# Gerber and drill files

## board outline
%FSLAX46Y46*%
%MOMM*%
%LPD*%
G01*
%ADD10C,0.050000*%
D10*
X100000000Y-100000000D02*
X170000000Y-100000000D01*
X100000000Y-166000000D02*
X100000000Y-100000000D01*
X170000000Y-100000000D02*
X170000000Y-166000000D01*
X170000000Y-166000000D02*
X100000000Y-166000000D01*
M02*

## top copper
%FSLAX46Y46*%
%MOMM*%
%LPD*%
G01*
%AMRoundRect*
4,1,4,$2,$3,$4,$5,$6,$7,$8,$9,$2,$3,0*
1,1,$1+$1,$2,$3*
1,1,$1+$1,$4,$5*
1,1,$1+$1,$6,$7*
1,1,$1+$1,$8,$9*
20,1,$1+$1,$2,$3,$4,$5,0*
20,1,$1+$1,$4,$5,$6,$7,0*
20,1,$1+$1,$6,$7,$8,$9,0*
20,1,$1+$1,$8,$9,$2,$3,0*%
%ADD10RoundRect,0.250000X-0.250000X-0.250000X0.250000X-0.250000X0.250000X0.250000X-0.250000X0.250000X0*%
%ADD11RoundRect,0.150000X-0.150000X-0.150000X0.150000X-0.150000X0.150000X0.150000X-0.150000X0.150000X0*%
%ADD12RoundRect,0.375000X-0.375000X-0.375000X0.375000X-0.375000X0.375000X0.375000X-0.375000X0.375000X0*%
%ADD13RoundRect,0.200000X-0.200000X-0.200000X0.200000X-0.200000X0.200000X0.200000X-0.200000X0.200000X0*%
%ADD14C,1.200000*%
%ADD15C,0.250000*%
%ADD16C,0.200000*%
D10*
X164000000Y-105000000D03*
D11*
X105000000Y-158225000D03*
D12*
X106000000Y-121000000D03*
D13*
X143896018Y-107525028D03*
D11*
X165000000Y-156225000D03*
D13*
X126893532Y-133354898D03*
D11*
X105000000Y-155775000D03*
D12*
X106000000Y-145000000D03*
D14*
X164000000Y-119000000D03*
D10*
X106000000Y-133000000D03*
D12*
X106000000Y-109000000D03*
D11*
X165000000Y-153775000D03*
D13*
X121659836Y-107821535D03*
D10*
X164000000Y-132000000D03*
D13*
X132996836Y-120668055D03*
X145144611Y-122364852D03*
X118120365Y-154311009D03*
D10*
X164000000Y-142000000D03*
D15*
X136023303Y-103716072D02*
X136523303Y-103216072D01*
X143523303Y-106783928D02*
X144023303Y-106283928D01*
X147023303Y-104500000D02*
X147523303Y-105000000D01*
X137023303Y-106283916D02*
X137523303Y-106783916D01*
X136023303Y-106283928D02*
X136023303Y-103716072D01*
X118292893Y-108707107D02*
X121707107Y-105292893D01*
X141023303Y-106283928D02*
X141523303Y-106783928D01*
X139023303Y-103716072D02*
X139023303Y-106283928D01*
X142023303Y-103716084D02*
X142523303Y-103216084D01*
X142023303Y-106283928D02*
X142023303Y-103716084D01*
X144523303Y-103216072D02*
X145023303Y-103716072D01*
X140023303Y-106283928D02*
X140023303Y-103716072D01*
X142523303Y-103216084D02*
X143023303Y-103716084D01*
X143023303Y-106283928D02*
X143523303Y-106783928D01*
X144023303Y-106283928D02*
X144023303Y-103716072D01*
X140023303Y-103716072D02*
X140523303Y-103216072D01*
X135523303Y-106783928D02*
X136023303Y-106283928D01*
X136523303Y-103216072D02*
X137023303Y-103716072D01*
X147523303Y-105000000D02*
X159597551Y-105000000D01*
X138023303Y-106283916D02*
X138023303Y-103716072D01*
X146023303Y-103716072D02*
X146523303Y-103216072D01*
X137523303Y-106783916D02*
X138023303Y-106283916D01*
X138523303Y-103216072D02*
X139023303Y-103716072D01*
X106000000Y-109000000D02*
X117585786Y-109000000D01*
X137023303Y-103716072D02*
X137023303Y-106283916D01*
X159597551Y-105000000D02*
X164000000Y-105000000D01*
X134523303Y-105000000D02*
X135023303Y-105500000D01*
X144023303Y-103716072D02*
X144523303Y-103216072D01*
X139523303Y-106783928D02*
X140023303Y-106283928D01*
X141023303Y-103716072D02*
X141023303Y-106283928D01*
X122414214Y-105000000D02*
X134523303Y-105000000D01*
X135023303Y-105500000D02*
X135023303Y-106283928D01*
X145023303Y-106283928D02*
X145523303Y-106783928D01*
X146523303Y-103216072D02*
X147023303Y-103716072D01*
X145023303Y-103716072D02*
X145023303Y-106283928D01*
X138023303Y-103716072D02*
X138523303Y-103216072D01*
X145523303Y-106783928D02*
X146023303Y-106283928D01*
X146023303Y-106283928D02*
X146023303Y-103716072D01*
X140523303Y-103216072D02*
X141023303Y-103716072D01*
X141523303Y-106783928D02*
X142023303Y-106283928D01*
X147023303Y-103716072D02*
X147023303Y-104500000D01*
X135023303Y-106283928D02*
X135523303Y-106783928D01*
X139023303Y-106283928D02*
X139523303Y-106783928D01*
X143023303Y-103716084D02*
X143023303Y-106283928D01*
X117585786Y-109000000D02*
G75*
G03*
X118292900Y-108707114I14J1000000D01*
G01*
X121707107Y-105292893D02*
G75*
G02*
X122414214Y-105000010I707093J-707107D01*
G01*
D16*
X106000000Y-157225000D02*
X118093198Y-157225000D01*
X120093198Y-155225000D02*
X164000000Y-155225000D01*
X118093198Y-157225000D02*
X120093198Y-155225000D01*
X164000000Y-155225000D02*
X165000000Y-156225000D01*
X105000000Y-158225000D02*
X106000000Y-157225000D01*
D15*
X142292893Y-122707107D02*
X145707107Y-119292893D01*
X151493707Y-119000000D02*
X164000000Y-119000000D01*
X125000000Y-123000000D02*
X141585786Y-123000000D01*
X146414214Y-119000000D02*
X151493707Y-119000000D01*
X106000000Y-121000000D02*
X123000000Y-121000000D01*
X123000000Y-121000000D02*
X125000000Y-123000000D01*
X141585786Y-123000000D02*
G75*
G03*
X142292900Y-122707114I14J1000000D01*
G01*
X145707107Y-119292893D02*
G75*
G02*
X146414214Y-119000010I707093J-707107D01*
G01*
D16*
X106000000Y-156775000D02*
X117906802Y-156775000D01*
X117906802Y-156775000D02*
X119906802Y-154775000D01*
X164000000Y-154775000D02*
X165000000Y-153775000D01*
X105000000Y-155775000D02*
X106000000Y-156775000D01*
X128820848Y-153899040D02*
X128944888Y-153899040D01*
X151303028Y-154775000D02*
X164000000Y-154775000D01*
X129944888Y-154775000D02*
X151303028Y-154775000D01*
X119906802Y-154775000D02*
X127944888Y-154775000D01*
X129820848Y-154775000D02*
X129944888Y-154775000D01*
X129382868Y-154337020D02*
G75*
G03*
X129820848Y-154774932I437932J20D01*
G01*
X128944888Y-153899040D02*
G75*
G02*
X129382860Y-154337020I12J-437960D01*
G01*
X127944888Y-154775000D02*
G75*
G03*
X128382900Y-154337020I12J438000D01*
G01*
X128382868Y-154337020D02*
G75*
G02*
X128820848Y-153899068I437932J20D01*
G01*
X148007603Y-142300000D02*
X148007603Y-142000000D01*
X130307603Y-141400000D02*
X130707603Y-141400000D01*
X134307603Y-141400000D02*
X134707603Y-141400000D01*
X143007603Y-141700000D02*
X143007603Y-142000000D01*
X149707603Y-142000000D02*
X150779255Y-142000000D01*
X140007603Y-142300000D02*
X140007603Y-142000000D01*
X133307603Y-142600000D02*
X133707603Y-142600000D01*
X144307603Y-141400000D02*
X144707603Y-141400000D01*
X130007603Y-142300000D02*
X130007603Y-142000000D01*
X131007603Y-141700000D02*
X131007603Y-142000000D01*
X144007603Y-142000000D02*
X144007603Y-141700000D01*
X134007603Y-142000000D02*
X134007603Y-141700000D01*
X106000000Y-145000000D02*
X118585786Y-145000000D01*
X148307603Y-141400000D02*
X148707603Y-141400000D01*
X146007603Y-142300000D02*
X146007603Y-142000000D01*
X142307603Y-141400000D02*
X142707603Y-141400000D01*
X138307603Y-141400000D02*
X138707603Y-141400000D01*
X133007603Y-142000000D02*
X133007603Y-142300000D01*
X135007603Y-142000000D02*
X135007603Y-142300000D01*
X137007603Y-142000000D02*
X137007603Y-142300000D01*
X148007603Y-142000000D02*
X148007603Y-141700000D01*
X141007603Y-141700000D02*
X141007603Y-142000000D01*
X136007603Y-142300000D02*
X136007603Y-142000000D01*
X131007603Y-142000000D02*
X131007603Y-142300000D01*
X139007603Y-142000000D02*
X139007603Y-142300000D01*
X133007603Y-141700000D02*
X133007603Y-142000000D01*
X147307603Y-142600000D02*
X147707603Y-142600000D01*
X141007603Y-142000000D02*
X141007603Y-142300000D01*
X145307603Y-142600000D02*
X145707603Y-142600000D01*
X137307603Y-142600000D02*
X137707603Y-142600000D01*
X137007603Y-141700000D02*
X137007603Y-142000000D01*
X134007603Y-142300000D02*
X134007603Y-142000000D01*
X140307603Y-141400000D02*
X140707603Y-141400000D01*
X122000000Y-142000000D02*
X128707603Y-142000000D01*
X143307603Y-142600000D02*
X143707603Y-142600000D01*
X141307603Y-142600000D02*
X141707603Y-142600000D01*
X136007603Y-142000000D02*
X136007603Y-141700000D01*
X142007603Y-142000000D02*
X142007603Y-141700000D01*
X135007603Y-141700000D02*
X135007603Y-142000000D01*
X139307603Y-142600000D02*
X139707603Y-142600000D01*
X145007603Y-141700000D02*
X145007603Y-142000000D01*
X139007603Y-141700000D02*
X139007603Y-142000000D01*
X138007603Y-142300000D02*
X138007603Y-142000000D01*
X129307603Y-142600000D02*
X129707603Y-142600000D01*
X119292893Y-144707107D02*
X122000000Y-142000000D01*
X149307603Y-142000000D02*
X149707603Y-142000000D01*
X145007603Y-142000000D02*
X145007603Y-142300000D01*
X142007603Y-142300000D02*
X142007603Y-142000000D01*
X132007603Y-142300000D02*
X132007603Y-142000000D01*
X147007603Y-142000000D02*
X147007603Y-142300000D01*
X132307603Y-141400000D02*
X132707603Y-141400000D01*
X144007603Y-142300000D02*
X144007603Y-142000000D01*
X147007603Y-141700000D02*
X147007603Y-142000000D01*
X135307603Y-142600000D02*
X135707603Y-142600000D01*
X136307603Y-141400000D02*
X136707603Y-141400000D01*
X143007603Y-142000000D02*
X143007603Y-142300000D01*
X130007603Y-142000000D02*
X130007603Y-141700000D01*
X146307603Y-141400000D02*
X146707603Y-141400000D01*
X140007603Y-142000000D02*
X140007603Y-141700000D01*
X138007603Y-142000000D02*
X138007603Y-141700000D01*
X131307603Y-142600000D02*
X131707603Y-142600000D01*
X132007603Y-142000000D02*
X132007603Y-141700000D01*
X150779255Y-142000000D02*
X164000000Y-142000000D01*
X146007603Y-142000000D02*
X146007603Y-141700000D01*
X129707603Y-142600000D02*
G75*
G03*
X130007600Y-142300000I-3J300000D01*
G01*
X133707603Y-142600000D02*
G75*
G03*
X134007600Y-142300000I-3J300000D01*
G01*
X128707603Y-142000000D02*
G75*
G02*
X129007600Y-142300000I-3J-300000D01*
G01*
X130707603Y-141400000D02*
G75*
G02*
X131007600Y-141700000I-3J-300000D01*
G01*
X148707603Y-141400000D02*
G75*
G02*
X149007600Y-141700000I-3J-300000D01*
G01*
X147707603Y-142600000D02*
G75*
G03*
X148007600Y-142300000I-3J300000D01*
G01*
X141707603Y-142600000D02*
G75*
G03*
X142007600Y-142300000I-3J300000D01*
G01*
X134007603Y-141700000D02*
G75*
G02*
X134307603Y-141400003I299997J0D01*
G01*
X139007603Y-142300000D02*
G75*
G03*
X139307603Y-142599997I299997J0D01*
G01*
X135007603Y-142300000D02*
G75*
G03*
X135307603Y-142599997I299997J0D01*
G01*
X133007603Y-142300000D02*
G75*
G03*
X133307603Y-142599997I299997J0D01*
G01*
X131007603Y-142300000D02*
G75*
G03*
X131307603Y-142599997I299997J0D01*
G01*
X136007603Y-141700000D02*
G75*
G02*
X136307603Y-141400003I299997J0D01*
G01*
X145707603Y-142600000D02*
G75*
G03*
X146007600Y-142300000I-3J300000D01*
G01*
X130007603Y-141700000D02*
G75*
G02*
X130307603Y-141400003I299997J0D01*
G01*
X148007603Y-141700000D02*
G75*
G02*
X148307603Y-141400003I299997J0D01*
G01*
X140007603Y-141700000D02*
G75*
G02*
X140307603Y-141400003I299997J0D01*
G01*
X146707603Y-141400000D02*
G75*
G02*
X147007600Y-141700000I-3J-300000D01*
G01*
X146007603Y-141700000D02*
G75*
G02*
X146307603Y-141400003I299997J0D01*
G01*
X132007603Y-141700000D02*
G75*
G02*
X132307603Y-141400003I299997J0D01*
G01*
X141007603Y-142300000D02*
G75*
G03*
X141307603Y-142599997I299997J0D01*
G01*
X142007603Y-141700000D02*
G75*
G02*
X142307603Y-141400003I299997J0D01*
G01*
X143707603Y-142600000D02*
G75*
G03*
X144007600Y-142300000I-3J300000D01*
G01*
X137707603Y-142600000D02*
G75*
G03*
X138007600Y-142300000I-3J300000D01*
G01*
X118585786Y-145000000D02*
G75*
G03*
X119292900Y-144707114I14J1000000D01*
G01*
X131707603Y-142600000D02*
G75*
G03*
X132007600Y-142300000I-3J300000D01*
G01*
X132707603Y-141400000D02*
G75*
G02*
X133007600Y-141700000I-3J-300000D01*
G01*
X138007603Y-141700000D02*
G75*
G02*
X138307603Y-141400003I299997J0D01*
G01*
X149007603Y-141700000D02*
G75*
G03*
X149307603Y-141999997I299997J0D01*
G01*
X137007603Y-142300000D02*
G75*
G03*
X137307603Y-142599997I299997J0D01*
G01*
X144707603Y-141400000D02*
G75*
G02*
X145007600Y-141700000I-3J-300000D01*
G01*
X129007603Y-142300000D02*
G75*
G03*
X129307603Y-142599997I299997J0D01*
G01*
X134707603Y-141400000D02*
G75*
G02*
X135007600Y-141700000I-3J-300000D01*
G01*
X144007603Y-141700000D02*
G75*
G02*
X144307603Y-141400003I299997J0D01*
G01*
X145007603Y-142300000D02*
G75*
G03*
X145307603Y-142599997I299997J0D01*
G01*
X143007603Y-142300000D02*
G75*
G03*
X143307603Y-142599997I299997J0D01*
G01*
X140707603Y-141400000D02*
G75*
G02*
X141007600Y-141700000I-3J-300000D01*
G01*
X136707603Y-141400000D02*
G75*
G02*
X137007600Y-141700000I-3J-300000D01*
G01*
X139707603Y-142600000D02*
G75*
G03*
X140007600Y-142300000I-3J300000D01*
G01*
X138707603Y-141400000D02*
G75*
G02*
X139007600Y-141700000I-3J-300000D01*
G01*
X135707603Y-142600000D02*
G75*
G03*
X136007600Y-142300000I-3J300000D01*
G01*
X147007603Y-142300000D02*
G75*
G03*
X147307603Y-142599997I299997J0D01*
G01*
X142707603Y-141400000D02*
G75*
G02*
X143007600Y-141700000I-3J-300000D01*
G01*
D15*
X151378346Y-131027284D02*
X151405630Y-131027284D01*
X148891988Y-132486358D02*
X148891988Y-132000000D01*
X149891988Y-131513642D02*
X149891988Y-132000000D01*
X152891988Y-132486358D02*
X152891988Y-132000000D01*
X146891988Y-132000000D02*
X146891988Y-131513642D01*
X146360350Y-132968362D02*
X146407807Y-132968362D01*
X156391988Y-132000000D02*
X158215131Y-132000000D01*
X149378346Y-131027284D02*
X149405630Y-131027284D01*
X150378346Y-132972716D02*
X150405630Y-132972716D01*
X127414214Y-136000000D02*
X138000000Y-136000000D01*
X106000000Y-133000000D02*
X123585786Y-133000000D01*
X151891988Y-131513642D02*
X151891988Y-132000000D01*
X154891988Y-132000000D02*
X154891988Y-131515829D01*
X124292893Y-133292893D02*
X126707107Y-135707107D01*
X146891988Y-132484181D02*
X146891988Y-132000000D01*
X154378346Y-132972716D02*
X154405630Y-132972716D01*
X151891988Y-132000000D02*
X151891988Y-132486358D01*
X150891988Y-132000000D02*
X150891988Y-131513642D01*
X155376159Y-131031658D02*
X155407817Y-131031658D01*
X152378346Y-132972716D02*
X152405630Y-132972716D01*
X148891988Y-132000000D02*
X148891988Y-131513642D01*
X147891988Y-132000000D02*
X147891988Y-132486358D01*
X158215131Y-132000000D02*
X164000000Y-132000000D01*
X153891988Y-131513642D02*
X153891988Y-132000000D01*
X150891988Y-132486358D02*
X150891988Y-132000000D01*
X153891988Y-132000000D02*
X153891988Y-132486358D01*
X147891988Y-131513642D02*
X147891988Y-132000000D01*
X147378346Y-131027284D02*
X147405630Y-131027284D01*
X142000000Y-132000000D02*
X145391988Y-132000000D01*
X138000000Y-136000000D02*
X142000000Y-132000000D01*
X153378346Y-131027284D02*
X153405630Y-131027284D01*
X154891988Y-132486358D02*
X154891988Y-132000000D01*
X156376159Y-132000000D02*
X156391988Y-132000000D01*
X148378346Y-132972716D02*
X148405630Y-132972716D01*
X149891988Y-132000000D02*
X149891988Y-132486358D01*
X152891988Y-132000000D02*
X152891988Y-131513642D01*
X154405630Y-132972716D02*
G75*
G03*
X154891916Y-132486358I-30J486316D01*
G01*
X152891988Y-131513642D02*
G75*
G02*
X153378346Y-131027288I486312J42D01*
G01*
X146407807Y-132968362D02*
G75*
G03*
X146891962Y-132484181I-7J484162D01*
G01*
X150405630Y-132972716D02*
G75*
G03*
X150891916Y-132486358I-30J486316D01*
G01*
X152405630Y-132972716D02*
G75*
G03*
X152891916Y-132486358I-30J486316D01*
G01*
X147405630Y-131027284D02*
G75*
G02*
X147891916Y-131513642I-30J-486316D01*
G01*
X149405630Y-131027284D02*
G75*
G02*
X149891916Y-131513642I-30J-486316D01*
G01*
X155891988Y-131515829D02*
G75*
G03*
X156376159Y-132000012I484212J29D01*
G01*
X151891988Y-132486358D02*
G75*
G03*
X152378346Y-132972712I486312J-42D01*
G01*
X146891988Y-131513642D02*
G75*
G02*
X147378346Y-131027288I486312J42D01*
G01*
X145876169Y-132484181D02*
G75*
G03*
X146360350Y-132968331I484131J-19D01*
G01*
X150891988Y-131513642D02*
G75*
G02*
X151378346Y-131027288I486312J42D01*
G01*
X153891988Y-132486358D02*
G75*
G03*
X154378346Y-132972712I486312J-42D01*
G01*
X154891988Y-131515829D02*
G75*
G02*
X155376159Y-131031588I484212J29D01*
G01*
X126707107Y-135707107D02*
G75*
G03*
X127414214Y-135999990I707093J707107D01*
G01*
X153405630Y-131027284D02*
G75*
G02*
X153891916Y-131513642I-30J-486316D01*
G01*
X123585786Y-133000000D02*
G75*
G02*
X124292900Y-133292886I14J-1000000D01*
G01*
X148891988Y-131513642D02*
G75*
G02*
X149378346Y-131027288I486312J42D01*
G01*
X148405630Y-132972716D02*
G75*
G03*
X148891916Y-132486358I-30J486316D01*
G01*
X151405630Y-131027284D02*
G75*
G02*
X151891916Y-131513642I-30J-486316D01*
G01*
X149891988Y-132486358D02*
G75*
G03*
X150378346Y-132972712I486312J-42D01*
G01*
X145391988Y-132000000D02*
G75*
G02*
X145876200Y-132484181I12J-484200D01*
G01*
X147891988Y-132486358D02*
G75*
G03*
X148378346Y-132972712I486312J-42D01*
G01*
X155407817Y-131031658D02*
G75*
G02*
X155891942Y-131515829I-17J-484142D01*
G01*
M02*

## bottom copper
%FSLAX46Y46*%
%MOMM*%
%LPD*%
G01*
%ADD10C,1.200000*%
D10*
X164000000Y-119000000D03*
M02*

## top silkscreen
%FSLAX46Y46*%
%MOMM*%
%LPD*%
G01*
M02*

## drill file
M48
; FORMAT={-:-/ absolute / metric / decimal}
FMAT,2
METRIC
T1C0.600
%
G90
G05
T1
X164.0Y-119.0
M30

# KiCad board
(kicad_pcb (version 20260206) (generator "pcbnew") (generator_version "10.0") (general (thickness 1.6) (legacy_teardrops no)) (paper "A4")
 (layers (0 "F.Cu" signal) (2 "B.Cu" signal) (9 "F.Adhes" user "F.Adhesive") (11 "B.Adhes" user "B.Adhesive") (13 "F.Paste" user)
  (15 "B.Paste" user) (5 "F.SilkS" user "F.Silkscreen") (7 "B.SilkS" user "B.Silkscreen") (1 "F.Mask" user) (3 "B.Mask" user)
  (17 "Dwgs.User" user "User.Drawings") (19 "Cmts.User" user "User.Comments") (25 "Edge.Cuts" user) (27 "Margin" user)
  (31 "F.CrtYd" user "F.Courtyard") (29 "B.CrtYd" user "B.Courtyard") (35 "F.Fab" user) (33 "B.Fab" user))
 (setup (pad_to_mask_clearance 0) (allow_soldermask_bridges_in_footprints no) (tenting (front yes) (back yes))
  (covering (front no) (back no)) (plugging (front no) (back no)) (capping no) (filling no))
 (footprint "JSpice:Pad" (layer "F.Cu") (at 164 105)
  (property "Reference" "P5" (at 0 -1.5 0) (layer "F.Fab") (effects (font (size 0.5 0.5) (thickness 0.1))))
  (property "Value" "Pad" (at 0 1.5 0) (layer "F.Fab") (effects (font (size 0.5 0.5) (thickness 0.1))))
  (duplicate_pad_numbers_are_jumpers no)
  (pad "1" smd roundrect (at 0 0) (size 1 1) (layers "F.Cu" "F.Mask") (roundrect_rratio 0.25) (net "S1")))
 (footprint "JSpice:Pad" (layer "F.Cu") (at 105 158.225)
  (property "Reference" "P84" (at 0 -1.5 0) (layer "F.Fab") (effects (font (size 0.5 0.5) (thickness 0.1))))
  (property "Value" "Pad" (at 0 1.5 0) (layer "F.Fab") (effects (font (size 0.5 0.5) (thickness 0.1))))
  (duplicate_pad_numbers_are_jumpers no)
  (pad "1" smd roundrect (at 0 0) (size 0.6 0.6) (layers "F.Cu" "F.Mask") (roundrect_rratio 0.25) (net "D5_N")))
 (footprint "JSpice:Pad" (layer "F.Cu") (at 106 121)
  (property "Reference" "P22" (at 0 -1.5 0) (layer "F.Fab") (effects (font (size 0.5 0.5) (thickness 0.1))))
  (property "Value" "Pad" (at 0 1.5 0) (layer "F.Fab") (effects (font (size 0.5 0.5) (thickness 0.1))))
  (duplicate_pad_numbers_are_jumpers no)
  (pad "1" smd roundrect (at 0 0) (size 1.5 1.5) (layers "F.Cu" "F.Mask") (roundrect_rratio 0.25) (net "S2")))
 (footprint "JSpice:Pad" (layer "F.Cu") (at 143.896018 107.525028)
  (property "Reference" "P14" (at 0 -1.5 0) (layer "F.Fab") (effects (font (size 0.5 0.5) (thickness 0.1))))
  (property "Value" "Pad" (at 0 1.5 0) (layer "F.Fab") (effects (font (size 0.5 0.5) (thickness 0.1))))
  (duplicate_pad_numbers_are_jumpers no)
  (pad "1" smd roundrect (at 0 0) (size 0.8 0.8) (layers "F.Cu" "F.Mask") (roundrect_rratio 0.25) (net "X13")))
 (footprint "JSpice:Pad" (layer "F.Cu") (at 165 156.225)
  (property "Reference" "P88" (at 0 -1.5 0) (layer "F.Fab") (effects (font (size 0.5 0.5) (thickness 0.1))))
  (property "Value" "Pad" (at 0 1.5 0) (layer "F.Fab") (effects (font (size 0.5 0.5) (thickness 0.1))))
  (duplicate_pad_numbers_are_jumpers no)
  (pad "1" smd roundrect (at 0 0) (size 0.6 0.6) (layers "F.Cu" "F.Mask") (roundrect_rratio 0.25) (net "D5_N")))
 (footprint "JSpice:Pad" (layer "F.Cu") (at 126.893532 133.354898)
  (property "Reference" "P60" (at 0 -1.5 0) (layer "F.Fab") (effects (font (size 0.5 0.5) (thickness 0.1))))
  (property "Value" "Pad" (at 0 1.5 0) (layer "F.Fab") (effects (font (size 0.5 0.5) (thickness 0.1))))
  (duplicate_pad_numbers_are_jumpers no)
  (pad "1" smd roundrect (at 0 0) (size 0.8 0.8) (layers "F.Cu" "F.Mask") (roundrect_rratio 0.25) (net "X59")))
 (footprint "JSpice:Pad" (layer "F.Cu") (at 105 155.775)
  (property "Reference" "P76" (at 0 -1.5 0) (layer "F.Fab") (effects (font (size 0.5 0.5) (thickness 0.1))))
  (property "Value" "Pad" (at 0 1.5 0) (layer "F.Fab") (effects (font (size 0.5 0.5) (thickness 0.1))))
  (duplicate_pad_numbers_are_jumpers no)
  (pad "1" smd roundrect (at 0 0) (size 0.6 0.6) (layers "F.Cu" "F.Mask") (roundrect_rratio 0.25) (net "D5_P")))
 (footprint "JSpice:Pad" (layer "F.Cu") (at 106 145)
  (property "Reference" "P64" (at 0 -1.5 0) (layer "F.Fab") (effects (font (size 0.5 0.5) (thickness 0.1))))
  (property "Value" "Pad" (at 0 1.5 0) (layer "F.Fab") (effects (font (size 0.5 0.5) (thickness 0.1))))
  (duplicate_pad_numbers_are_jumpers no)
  (pad "1" smd roundrect (at 0 0) (size 1.5 1.5) (layers "F.Cu" "F.Mask") (roundrect_rratio 0.25) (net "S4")))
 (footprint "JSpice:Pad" (layer "F.Cu") (at 164 119)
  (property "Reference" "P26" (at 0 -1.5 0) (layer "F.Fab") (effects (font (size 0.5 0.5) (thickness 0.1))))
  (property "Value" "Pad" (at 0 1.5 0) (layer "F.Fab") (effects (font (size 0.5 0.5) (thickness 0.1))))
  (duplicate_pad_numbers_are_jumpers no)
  (pad "1" thru_hole circle (at 0 0) (size 1.2 1.2) (drill 0.6) (layers "*.Cu" "*.Mask") (remove_unused_layers no) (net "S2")))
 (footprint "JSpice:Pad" (layer "F.Cu") (at 106 133)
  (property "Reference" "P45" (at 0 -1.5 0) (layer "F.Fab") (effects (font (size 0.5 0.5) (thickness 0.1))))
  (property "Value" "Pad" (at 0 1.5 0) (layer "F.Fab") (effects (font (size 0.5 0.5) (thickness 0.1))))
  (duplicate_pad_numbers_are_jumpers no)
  (pad "1" smd roundrect (at 0 0) (size 1 1) (layers "F.Cu" "F.Mask") (roundrect_rratio 0.25) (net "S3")))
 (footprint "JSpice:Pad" (layer "F.Cu") (at 106 109)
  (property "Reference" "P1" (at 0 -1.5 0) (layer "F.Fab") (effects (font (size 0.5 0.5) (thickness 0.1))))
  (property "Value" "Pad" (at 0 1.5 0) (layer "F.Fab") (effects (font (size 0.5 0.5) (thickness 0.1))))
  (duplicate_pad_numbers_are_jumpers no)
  (pad "1" smd roundrect (at 0 0) (size 1.5 1.5) (layers "F.Cu" "F.Mask") (roundrect_rratio 0.25) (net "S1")))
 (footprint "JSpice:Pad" (layer "F.Cu") (at 165 153.775)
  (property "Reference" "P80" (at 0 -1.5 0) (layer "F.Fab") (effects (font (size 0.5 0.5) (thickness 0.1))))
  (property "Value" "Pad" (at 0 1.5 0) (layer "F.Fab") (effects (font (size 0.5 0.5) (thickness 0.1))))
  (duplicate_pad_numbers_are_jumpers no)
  (pad "1" smd roundrect (at 0 0) (size 0.6 0.6) (layers "F.Cu" "F.Mask") (roundrect_rratio 0.25) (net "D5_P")))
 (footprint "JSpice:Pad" (layer "F.Cu") (at 121.659836 107.821535)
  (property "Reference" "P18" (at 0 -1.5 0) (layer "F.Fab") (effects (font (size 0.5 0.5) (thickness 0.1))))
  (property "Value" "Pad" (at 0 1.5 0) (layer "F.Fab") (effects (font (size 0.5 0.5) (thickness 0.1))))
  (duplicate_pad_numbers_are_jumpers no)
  (pad "1" smd roundrect (at 0 0) (size 0.8 0.8) (layers "F.Cu" "F.Mask") (roundrect_rratio 0.25) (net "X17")))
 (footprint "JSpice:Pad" (layer "F.Cu") (at 164 132)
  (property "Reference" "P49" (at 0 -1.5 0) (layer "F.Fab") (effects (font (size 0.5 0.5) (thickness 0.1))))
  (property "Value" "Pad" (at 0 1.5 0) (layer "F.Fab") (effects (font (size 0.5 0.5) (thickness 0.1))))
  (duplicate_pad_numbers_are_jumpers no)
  (pad "1" smd roundrect (at 0 0) (size 1 1) (layers "F.Cu" "F.Mask") (roundrect_rratio 0.25) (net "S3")))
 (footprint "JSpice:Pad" (layer "F.Cu") (at 132.996836 120.668055)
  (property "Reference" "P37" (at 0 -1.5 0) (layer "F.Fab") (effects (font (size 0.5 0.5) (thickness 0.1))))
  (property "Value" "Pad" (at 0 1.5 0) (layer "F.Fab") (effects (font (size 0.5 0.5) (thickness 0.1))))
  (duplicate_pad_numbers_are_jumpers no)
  (pad "1" smd roundrect (at 0 0) (size 0.8 0.8) (layers "F.Cu" "F.Mask") (roundrect_rratio 0.25) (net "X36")))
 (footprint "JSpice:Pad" (layer "F.Cu") (at 145.144611 122.364852)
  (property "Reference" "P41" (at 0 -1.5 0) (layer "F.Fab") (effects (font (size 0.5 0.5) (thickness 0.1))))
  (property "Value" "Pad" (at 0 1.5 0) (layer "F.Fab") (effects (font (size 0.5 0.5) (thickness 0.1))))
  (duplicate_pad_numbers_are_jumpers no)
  (pad "1" smd roundrect (at 0 0) (size 0.8 0.8) (layers "F.Cu" "F.Mask") (roundrect_rratio 0.25) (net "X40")))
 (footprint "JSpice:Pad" (layer "F.Cu") (at 118.120365 154.311009)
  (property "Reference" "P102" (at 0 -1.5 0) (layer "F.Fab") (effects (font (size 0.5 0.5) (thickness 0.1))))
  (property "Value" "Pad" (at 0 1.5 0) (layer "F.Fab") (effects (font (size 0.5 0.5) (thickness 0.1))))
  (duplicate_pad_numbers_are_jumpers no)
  (pad "1" smd roundrect (at 0 0) (size 0.8 0.8) (layers "F.Cu" "F.Mask") (roundrect_rratio 0.25) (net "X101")))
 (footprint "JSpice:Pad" (layer "F.Cu") (at 164 142)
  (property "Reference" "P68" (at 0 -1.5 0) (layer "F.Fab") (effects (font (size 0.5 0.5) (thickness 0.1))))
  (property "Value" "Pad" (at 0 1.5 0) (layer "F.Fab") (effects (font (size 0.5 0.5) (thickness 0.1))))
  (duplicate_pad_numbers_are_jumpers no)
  (pad "1" smd roundrect (at 0 0) (size 1 1) (layers "F.Cu" "F.Mask") (roundrect_rratio 0.25) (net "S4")))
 (gr_line (start 100 100) (end 170 100) (stroke (width 0.05) (type default)) (layer "Edge.Cuts"))
 (gr_line (start 100 166) (end 100 100) (stroke (width 0.05) (type default)) (layer "Edge.Cuts"))
 (gr_line (start 170 100) (end 170 166) (stroke (width 0.05) (type default)) (layer "Edge.Cuts"))
 (gr_line (start 170 166) (end 100 166) (stroke (width 0.05) (type default)) (layer "Edge.Cuts"))
 (segment (start 136.023303 103.716072) (end 136.523303 103.216072) (width 0.25) (layer "F.Cu") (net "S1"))
 (segment (start 143.523303 106.783928) (end 144.023303 106.283928) (width 0.25) (layer "F.Cu") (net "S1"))
 (segment (start 147.023303 104.5) (end 147.523303 105) (width 0.25) (layer "F.Cu") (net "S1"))
 (segment (start 137.023303 106.283916) (end 137.523303 106.783916) (width 0.25) (layer "F.Cu") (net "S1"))
 (segment (start 136.023303 106.283928) (end 136.023303 103.716072) (width 0.25) (layer "F.Cu") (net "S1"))
 (segment (start 118.292893 108.707107) (end 121.707107 105.292893) (width 0.25) (layer "F.Cu") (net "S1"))
 (segment (start 141.023303 106.283928) (end 141.523303 106.783928) (width 0.25) (layer "F.Cu") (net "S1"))
 (segment (start 139.023303 103.716072) (end 139.023303 106.283928) (width 0.25) (layer "F.Cu") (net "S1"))
 (segment (start 142.023303 103.716084) (end 142.523303 103.216084) (width 0.25) (layer "F.Cu") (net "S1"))
 (segment (start 142.023303 106.283928) (end 142.023303 103.716084) (width 0.25) (layer "F.Cu") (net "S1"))
 (segment (start 144.523303 103.216072) (end 145.023303 103.716072) (width 0.25) (layer "F.Cu") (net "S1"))
 (segment (start 140.023303 106.283928) (end 140.023303 103.716072) (width 0.25) (layer "F.Cu") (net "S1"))
 (segment (start 142.523303 103.216084) (end 143.023303 103.716084) (width 0.25) (layer "F.Cu") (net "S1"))
 (segment (start 143.023303 106.283928) (end 143.523303 106.783928) (width 0.25) (layer "F.Cu") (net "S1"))
 (segment (start 144.023303 106.283928) (end 144.023303 103.716072) (width 0.25) (layer "F.Cu") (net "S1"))
 (segment (start 140.023303 103.716072) (end 140.523303 103.216072) (width 0.25) (layer "F.Cu") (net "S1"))
 (segment (start 135.523303 106.783928) (end 136.023303 106.283928) (width 0.25) (layer "F.Cu") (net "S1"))
 (segment (start 136.523303 103.216072) (end 137.023303 103.716072) (width 0.25) (layer "F.Cu") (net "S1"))
 (segment (start 147.523303 105) (end 159.597551 105) (width 0.25) (layer "F.Cu") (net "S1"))
 (segment (start 138.023303 106.283916) (end 138.023303 103.716072) (width 0.25) (layer "F.Cu") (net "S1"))
 (segment (start 146.023303 103.716072) (end 146.523303 103.216072) (width 0.25) (layer "F.Cu") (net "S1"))
 (segment (start 137.523303 106.783916) (end 138.023303 106.283916) (width 0.25) (layer "F.Cu") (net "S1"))
 (segment (start 138.523303 103.216072) (end 139.023303 103.716072) (width 0.25) (layer "F.Cu") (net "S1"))
 (segment (start 106 109) (end 117.585786 109) (width 0.25) (layer "F.Cu") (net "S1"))
 (segment (start 137.023303 103.716072) (end 137.023303 106.283916) (width 0.25) (layer "F.Cu") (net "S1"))
 (segment (start 159.597551 105) (end 164 105) (width 0.25) (layer "F.Cu") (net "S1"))
 (segment (start 134.523303 105) (end 135.023303 105.5) (width 0.25) (layer "F.Cu") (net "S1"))
 (segment (start 144.023303 103.716072) (end 144.523303 103.216072) (width 0.25) (layer "F.Cu") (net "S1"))
 (segment (start 139.523303 106.783928) (end 140.023303 106.283928) (width 0.25) (layer "F.Cu") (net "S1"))
 (segment (start 141.023303 103.716072) (end 141.023303 106.283928) (width 0.25) (layer "F.Cu") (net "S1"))
 (segment (start 122.414214 105) (end 134.523303 105) (width 0.25) (layer "F.Cu") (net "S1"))
 (segment (start 135.023303 105.5) (end 135.023303 106.283928) (width 0.25) (layer "F.Cu") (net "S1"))
 (segment (start 145.023303 106.283928) (end 145.523303 106.783928) (width 0.25) (layer "F.Cu") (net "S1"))
 (segment (start 146.523303 103.216072) (end 147.023303 103.716072) (width 0.25) (layer "F.Cu") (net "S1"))
 (segment (start 145.023303 103.716072) (end 145.023303 106.283928) (width 0.25) (layer "F.Cu") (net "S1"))
 (segment (start 138.023303 103.716072) (end 138.523303 103.216072) (width 0.25) (layer "F.Cu") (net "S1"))
 (segment (start 145.523303 106.783928) (end 146.023303 106.283928) (width 0.25) (layer "F.Cu") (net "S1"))
 (segment (start 146.023303 106.283928) (end 146.023303 103.716072) (width 0.25) (layer "F.Cu") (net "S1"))
 (segment (start 140.523303 103.216072) (end 141.023303 103.716072) (width 0.25) (layer "F.Cu") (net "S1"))
 (segment (start 141.523303 106.783928) (end 142.023303 106.283928) (width 0.25) (layer "F.Cu") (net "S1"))
 (segment (start 147.023303 103.716072) (end 147.023303 104.5) (width 0.25) (layer "F.Cu") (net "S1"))
 (segment (start 135.023303 106.283928) (end 135.523303 106.783928) (width 0.25) (layer "F.Cu") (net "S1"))
 (segment (start 139.023303 106.283928) (end 139.523303 106.783928) (width 0.25) (layer "F.Cu") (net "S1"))
 (segment (start 143.023303 103.716084) (end 143.023303 106.283928) (width 0.25) (layer "F.Cu") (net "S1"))
 (arc (start 117.585786 109) (mid 117.96847 108.92388) (end 118.292893 108.707107) (width 0.25) (layer "F.Cu") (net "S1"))
 (arc (start 121.707107 105.292893) (mid 122.03153 105.07612) (end 122.414214 105) (width 0.25) (layer "F.Cu") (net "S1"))
 (segment (start 106 157.225) (end 118.093198 157.225) (width 0.2) (layer "F.Cu") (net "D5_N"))
 (segment (start 120.093198 155.225) (end 164 155.225) (width 0.2) (layer "F.Cu") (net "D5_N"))
 (segment (start 118.093198 157.225) (end 120.093198 155.225) (width 0.2) (layer "F.Cu") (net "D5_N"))
 (segment (start 164 155.225) (end 165 156.225) (width 0.2) (layer "F.Cu") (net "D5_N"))
 (segment (start 105 158.225) (end 106 157.225) (width 0.2) (layer "F.Cu") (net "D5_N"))
 (segment (start 142.292893 122.707107) (end 145.707107 119.292893) (width 0.25) (layer "F.Cu") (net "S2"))
 (segment (start 151.493707 119) (end 164 119) (width 0.25) (layer "F.Cu") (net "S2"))
 (segment (start 125 123) (end 141.585786 123) (width 0.25) (layer "F.Cu") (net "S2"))
 (segment (start 146.414214 119) (end 151.493707 119) (width 0.25) (layer "F.Cu") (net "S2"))
 (segment (start 106 121) (end 123 121) (width 0.25) (layer "F.Cu") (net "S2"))
 (segment (start 123 121) (end 125 123) (width 0.25) (layer "F.Cu") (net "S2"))
 (arc (start 141.585786 123) (mid 141.96847 122.92388) (end 142.292893 122.707107) (width 0.25) (layer "F.Cu") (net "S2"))
 (arc (start 145.707107 119.292893) (mid 146.03153 119.07612) (end 146.414214 119) (width 0.25) (layer "F.Cu") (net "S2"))
 (segment (start 106 156.775) (end 117.906802 156.775) (width 0.2) (layer "F.Cu") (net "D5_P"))
 (segment (start 117.906802 156.775) (end 119.906802 154.775) (width 0.2) (layer "F.Cu") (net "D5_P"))
 (segment (start 164 154.775) (end 165 153.775) (width 0.2) (layer "F.Cu") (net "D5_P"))
 (segment (start 105 155.775) (end 106 156.775) (width 0.2) (layer "F.Cu") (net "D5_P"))
 (segment (start 128.820848 153.89904) (end 128.944888 153.89904) (width 0.2) (layer "F.Cu") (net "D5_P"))
 (segment (start 151.303028 154.775) (end 164 154.775) (width 0.2) (layer "F.Cu") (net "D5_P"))
 (segment (start 129.944888 154.775) (end 151.303028 154.775) (width 0.2) (layer "F.Cu") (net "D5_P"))
 (segment (start 119.906802 154.775) (end 127.944888 154.775) (width 0.2) (layer "F.Cu") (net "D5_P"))
 (segment (start 129.820848 154.775) (end 129.944888 154.775) (width 0.2) (layer "F.Cu") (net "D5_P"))
 (arc (start 129.382868 154.33702) (mid 129.511149 154.646719) (end 129.820848 154.775) (width 0.2) (layer "F.Cu") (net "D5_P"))
 (arc (start 128.944888 153.89904) (mid 129.254587 154.027321) (end 129.382868 154.33702) (width 0.2) (layer "F.Cu") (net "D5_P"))
 (arc (start 127.944888 154.775) (mid 128.254587 154.646719) (end 128.382868 154.33702) (width 0.2) (layer "F.Cu") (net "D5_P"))
 (arc (start 128.382868 154.33702) (mid 128.511149 154.027321) (end 128.820848 153.89904) (width 0.2) (layer "F.Cu") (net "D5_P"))
 (segment (start 148.007603 142.3) (end 148.007603 142) (width 0.2) (layer "F.Cu") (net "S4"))
 (segment (start 130.307603 141.4) (end 130.707603 141.4) (width 0.2) (layer "F.Cu") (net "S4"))
 (segment (start 134.307603 141.4) (end 134.707603 141.4) (width 0.2) (layer "F.Cu") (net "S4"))
 (segment (start 143.007603 141.7) (end 143.007603 142) (width 0.2) (layer "F.Cu") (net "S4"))
 (segment (start 149.707603 142) (end 150.779255 142) (width 0.2) (layer "F.Cu") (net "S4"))
 (segment (start 140.007603 142.3) (end 140.007603 142) (width 0.2) (layer "F.Cu") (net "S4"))
 (segment (start 133.307603 142.6) (end 133.707603 142.6) (width 0.2) (layer "F.Cu") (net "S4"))
 (segment (start 144.307603 141.4) (end 144.707603 141.4) (width 0.2) (layer "F.Cu") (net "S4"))
 (segment (start 130.007603 142.3) (end 130.007603 142) (width 0.2) (layer "F.Cu") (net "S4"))
 (segment (start 131.007603 141.7) (end 131.007603 142) (width 0.2) (layer "F.Cu") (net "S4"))
 (segment (start 144.007603 142) (end 144.007603 141.7) (width 0.2) (layer "F.Cu") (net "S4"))
 (segment (start 134.007603 142) (end 134.007603 141.7) (width 0.2) (layer "F.Cu") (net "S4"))
 (segment (start 106 145) (end 118.585786 145) (width 0.2) (layer "F.Cu") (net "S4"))
 (segment (start 148.307603 141.4) (end 148.707603 141.4) (width 0.2) (layer "F.Cu") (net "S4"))
 (segment (start 146.007603 142.3) (end 146.007603 142) (width 0.2) (layer "F.Cu") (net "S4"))
 (segment (start 142.307603 141.4) (end 142.707603 141.4) (width 0.2) (layer "F.Cu") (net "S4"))
 (segment (start 138.307603 141.4) (end 138.707603 141.4) (width 0.2) (layer "F.Cu") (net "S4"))
 (segment (start 133.007603 142) (end 133.007603 142.3) (width 0.2) (layer "F.Cu") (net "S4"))
 (segment (start 135.007603 142) (end 135.007603 142.3) (width 0.2) (layer "F.Cu") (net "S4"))
 (segment (start 137.007603 142) (end 137.007603 142.3) (width 0.2) (layer "F.Cu") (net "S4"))
 (segment (start 148.007603 142) (end 148.007603 141.7) (width 0.2) (layer "F.Cu") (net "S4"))
 (segment (start 141.007603 141.7) (end 141.007603 142) (width 0.2) (layer "F.Cu") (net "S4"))
 (segment (start 136.007603 142.3) (end 136.007603 142) (width 0.2) (layer "F.Cu") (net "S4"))
 (segment (start 131.007603 142) (end 131.007603 142.3) (width 0.2) (layer "F.Cu") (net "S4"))
 (segment (start 139.007603 142) (end 139.007603 142.3) (width 0.2) (layer "F.Cu") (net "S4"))
 (segment (start 133.007603 141.7) (end 133.007603 142) (width 0.2) (layer "F.Cu") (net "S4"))
 (segment (start 147.307603 142.6) (end 147.707603 142.6) (width 0.2) (layer "F.Cu") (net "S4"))
 (segment (start 141.007603 142) (end 141.007603 142.3) (width 0.2) (layer "F.Cu") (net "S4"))
 (segment (start 145.307603 142.6) (end 145.707603 142.6) (width 0.2) (layer "F.Cu") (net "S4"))
 (segment (start 137.307603 142.6) (end 137.707603 142.6) (width 0.2) (layer "F.Cu") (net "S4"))
 (segment (start 137.007603 141.7) (end 137.007603 142) (width 0.2) (layer "F.Cu") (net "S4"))
 (segment (start 134.007603 142.3) (end 134.007603 142) (width 0.2) (layer "F.Cu") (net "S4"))
 (segment (start 140.307603 141.4) (end 140.707603 141.4) (width 0.2) (layer "F.Cu") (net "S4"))
 (segment (start 122 142) (end 128.707603 142) (width 0.2) (layer "F.Cu") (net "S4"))
 (segment (start 143.307603 142.6) (end 143.707603 142.6) (width 0.2) (layer "F.Cu") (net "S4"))
 (segment (start 141.307603 142.6) (end 141.707603 142.6) (width 0.2) (layer "F.Cu") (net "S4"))
 (segment (start 136.007603 142) (end 136.007603 141.7) (width 0.2) (layer "F.Cu") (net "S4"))
 (segment (start 142.007603 142) (end 142.007603 141.7) (width 0.2) (layer "F.Cu") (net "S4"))
 (segment (start 135.007603 141.7) (end 135.007603 142) (width 0.2) (layer "F.Cu") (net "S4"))
 (segment (start 139.307603 142.6) (end 139.707603 142.6) (width 0.2) (layer "F.Cu") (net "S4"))
 (segment (start 145.007603 141.7) (end 145.007603 142) (width 0.2) (layer "F.Cu") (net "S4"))
 (segment (start 139.007603 141.7) (end 139.007603 142) (width 0.2) (layer "F.Cu") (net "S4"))
 (segment (start 138.007603 142.3) (end 138.007603 142) (width 0.2) (layer "F.Cu") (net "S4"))
 (segment (start 129.307603 142.6) (end 129.707603 142.6) (width 0.2) (layer "F.Cu") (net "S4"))
 (segment (start 119.292893 144.707107) (end 122 142) (width 0.2) (layer "F.Cu") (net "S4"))
 (segment (start 149.307603 142) (end 149.707603 142) (width 0.2) (layer "F.Cu") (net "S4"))
 (segment (start 145.007603 142) (end 145.007603 142.3) (width 0.2) (layer "F.Cu") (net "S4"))
 (segment (start 142.007603 142.3) (end 142.007603 142) (width 0.2) (layer "F.Cu") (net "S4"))
 (segment (start 132.007603 142.3) (end 132.007603 142) (width 0.2) (layer "F.Cu") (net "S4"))
 (segment (start 147.007603 142) (end 147.007603 142.3) (width 0.2) (layer "F.Cu") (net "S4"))
 (segment (start 132.307603 141.4) (end 132.707603 141.4) (width 0.2) (layer "F.Cu") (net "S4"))
 (segment (start 144.007603 142.3) (end 144.007603 142) (width 0.2) (layer "F.Cu") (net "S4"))
 (segment (start 147.007603 141.7) (end 147.007603 142) (width 0.2) (layer "F.Cu") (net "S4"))
 (segment (start 135.307603 142.6) (end 135.707603 142.6) (width 0.2) (layer "F.Cu") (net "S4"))
 (segment (start 136.307603 141.4) (end 136.707603 141.4) (width 0.2) (layer "F.Cu") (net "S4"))
 (segment (start 143.007603 142) (end 143.007603 142.3) (width 0.2) (layer "F.Cu") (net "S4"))
 (segment (start 130.007603 142) (end 130.007603 141.7) (width 0.2) (layer "F.Cu") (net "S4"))
 (segment (start 146.307603 141.4) (end 146.707603 141.4) (width 0.2) (layer "F.Cu") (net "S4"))
 (segment (start 140.007603 142) (end 140.007603 141.7) (width 0.2) (layer "F.Cu") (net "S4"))
 (segment (start 138.007603 142) (end 138.007603 141.7) (width 0.2) (layer "F.Cu") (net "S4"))
 (segment (start 131.307603 142.6) (end 131.707603 142.6) (width 0.2) (layer "F.Cu") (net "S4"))
 (segment (start 132.007603 142) (end 132.007603 141.7) (width 0.2) (layer "F.Cu") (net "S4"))
 (segment (start 150.779255 142) (end 164 142) (width 0.2) (layer "F.Cu") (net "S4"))
 (segment (start 146.007603 142) (end 146.007603 141.7) (width 0.2) (layer "F.Cu") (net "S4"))
 (arc (start 129.707603 142.6) (mid 129.919735 142.512132) (end 130.007603 142.3) (width 0.2) (layer "F.Cu") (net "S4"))
 (arc (start 133.707603 142.6) (mid 133.919735 142.512132) (end 134.007603 142.3) (width 0.2) (layer "F.Cu") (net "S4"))
 (arc (start 128.707603 142) (mid 128.919735 142.087868) (end 129.007603 142.3) (width 0.2) (layer "F.Cu") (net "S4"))
 (arc (start 130.707603 141.4) (mid 130.919735 141.487868) (end 131.007603 141.7) (width 0.2) (layer "F.Cu") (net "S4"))
 (arc (start 148.707603 141.4) (mid 148.919735 141.487868) (end 149.007603 141.7) (width 0.2) (layer "F.Cu") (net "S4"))
 (arc (start 147.707603 142.6) (mid 147.919735 142.512132) (end 148.007603 142.3) (width 0.2) (layer "F.Cu") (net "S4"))
 (arc (start 141.707603 142.6) (mid 141.919735 142.512132) (end 142.007603 142.3) (width 0.2) (layer "F.Cu") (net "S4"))
 (arc (start 134.007603 141.7) (mid 134.095471 141.487868) (end 134.307603 141.4) (width 0.2) (layer "F.Cu") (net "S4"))
 (arc (start 139.007603 142.3) (mid 139.095471 142.512132) (end 139.307603 142.6) (width 0.2) (layer "F.Cu") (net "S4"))
 (arc (start 135.007603 142.3) (mid 135.095471 142.512132) (end 135.307603 142.6) (width 0.2) (layer "F.Cu") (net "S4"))
 (arc (start 133.007603 142.3) (mid 133.095471 142.512132) (end 133.307603 142.6) (width 0.2) (layer "F.Cu") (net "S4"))
 (arc (start 131.007603 142.3) (mid 131.095471 142.512132) (end 131.307603 142.6) (width 0.2) (layer "F.Cu") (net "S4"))
 (arc (start 136.007603 141.7) (mid 136.095471 141.487868) (end 136.307603 141.4) (width 0.2) (layer "F.Cu") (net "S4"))
 (arc (start 145.707603 142.6) (mid 145.919735 142.512132) (end 146.007603 142.3) (width 0.2) (layer "F.Cu") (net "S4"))
 (arc (start 130.007603 141.7) (mid 130.095471 141.487868) (end 130.307603 141.4) (width 0.2) (layer "F.Cu") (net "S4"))
 (arc (start 148.007603 141.7) (mid 148.095471 141.487868) (end 148.307603 141.4) (width 0.2) (layer "F.Cu") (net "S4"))
 (arc (start 140.007603 141.7) (mid 140.095471 141.487868) (end 140.307603 141.4) (width 0.2) (layer "F.Cu") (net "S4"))
 (arc (start 146.707603 141.4) (mid 146.919735 141.487868) (end 147.007603 141.7) (width 0.2) (layer "F.Cu") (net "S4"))
 (arc (start 146.007603 141.7) (mid 146.095471 141.487868) (end 146.307603 141.4) (width 0.2) (layer "F.Cu") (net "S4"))
 (arc (start 132.007603 141.7) (mid 132.095471 141.487868) (end 132.307603 141.4) (width 0.2) (layer "F.Cu") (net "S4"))
 (arc (start 141.007603 142.3) (mid 141.095471 142.512132) (end 141.307603 142.6) (width 0.2) (layer "F.Cu") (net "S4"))
 (arc (start 142.007603 141.7) (mid 142.095471 141.487868) (end 142.307603 141.4) (width 0.2) (layer "F.Cu") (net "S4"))
 (arc (start 143.707603 142.6) (mid 143.919735 142.512132) (end 144.007603 142.3) (width 0.2) (layer "F.Cu") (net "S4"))
 (arc (start 137.707603 142.6) (mid 137.919735 142.512132) (end 138.007603 142.3) (width 0.2) (layer "F.Cu") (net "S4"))
 (arc (start 118.585786 145) (mid 118.96847 144.92388) (end 119.292893 144.707107) (width 0.2) (layer "F.Cu") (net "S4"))
 (arc (start 131.707603 142.6) (mid 131.919735 142.512132) (end 132.007603 142.3) (width 0.2) (layer "F.Cu") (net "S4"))
 (arc (start 132.707603 141.4) (mid 132.919735 141.487868) (end 133.007603 141.7) (width 0.2) (layer "F.Cu") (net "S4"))
 (arc (start 138.007603 141.7) (mid 138.095471 141.487868) (end 138.307603 141.4) (width 0.2) (layer "F.Cu") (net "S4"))
 (arc (start 149.007603 141.7) (mid 149.095471 141.912132) (end 149.307603 142) (width 0.2) (layer "F.Cu") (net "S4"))
 (arc (start 137.007603 142.3) (mid 137.095471 142.512132) (end 137.307603 142.6) (width 0.2) (layer "F.Cu") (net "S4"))
 (arc (start 144.707603 141.4) (mid 144.919735 141.487868) (end 145.007603 141.7) (width 0.2) (layer "F.Cu") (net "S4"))
 (arc (start 129.007603 142.3) (mid 129.095471 142.512132) (end 129.307603 142.6) (width 0.2) (layer "F.Cu") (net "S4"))
 (arc (start 134.707603 141.4) (mid 134.919735 141.487868) (end 135.007603 141.7) (width 0.2) (layer "F.Cu") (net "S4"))
 (arc (start 144.007603 141.7) (mid 144.095471 141.487868) (end 144.307603 141.4) (width 0.2) (layer "F.Cu") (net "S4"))
 (arc (start 145.007603 142.3) (mid 145.095471 142.512132) (end 145.307603 142.6) (width 0.2) (layer "F.Cu") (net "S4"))
 (arc (start 143.007603 142.3) (mid 143.095471 142.512132) (end 143.307603 142.6) (width 0.2) (layer "F.Cu") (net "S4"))
 (arc (start 140.707603 141.4) (mid 140.919735 141.487868) (end 141.007603 141.7) (width 0.2) (layer "F.Cu") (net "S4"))
 (arc (start 136.707603 141.4) (mid 136.919735 141.487868) (end 137.007603 141.7) (width 0.2) (layer "F.Cu") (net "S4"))
 (arc (start 139.707603 142.6) (mid 139.919735 142.512132) (end 140.007603 142.3) (width 0.2) (layer "F.Cu") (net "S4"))
 (arc (start 138.707603 141.4) (mid 138.919735 141.487868) (end 139.007603 141.7) (width 0.2) (layer "F.Cu") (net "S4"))
 (arc (start 135.707603 142.6) (mid 135.919735 142.512132) (end 136.007603 142.3) (width 0.2) (layer "F.Cu") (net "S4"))
 (arc (start 147.007603 142.3) (mid 147.095471 142.512132) (end 147.307603 142.6) (width 0.2) (layer "F.Cu") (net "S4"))
 (arc (start 142.707603 141.4) (mid 142.919735 141.487868) (end 143.007603 141.7) (width 0.2) (layer "F.Cu") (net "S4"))
 (segment (start 151.378346 131.027284) (end 151.40563 131.027284) (width 0.25) (layer "F.Cu") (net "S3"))
 (segment (start 148.891988 132.486358) (end 148.891988 132) (width 0.25) (layer "F.Cu") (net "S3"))
 (segment (start 149.891988 131.513642) (end 149.891988 132) (width 0.25) (layer "F.Cu") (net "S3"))
 (segment (start 152.891988 132.486358) (end 152.891988 132) (width 0.25) (layer "F.Cu") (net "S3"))
 (segment (start 146.891988 132) (end 146.891988 131.513642) (width 0.25) (layer "F.Cu") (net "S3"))
 (segment (start 146.36035 132.968362) (end 146.407807 132.968362) (width 0.25) (layer "F.Cu") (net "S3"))
 (segment (start 156.391988 132) (end 158.215131 132) (width 0.25) (layer "F.Cu") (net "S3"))
 (segment (start 149.378346 131.027284) (end 149.40563 131.027284) (width 0.25) (layer "F.Cu") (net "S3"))
 (segment (start 150.378346 132.972716) (end 150.40563 132.972716) (width 0.25) (layer "F.Cu") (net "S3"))
 (segment (start 127.414214 136) (end 138 136) (width 0.25) (layer "F.Cu") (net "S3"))
 (segment (start 106 133) (end 123.585786 133) (width 0.25) (layer "F.Cu") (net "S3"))
 (segment (start 151.891988 131.513642) (end 151.891988 132) (width 0.25) (layer "F.Cu") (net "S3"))
 (segment (start 154.891988 132) (end 154.891988 131.515829) (width 0.25) (layer "F.Cu") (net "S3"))
 (segment (start 124.292893 133.292893) (end 126.707107 135.707107) (width 0.25) (layer "F.Cu") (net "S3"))
 (segment (start 146.891988 132.484181) (end 146.891988 132) (width 0.25) (layer "F.Cu") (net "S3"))
 (segment (start 154.378346 132.972716) (end 154.40563 132.972716) (width 0.25) (layer "F.Cu") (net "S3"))
 (segment (start 151.891988 132) (end 151.891988 132.486358) (width 0.25) (layer "F.Cu") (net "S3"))
 (segment (start 150.891988 132) (end 150.891988 131.513642) (width 0.25) (layer "F.Cu") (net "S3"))
 (segment (start 155.376159 131.031658) (end 155.407817 131.031658) (width 0.25) (layer "F.Cu") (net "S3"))
 (segment (start 152.378346 132.972716) (end 152.40563 132.972716) (width 0.25) (layer "F.Cu") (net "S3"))
 (segment (start 148.891988 132) (end 148.891988 131.513642) (width 0.25) (layer "F.Cu") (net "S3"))
 (segment (start 147.891988 132) (end 147.891988 132.486358) (width 0.25) (layer "F.Cu") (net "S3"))
 (segment (start 158.215131 132) (end 164 132) (width 0.25) (layer "F.Cu") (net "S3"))
 (segment (start 153.891988 131.513642) (end 153.891988 132) (width 0.25) (layer "F.Cu") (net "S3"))
 (segment (start 150.891988 132.486358) (end 150.891988 132) (width 0.25) (layer "F.Cu") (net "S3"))
 (segment (start 153.891988 132) (end 153.891988 132.486358) (width 0.25) (layer "F.Cu") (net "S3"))
 (segment (start 147.891988 131.513642) (end 147.891988 132) (width 0.25) (layer "F.Cu") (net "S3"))
 (segment (start 147.378346 131.027284) (end 147.40563 131.027284) (width 0.25) (layer "F.Cu") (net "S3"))
 (segment (start 142 132) (end 145.391988 132) (width 0.25) (layer "F.Cu") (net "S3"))
 (segment (start 138 136) (end 142 132) (width 0.25) (layer "F.Cu") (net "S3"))
 (segment (start 153.378346 131.027284) (end 153.40563 131.027284) (width 0.25) (layer "F.Cu") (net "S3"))
 (segment (start 154.891988 132.486358) (end 154.891988 132) (width 0.25) (layer "F.Cu") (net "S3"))
 (segment (start 156.376159 132) (end 156.391988 132) (width 0.25) (layer "F.Cu") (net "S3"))
 (segment (start 148.378346 132.972716) (end 148.40563 132.972716) (width 0.25) (layer "F.Cu") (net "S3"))
 (segment (start 149.891988 132) (end 149.891988 132.486358) (width 0.25) (layer "F.Cu") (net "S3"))
 (segment (start 152.891988 132) (end 152.891988 131.513642) (width 0.25) (layer "F.Cu") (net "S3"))
 (arc (start 154.40563 132.972716) (mid 154.749537 132.830265) (end 154.891988 132.486358) (width 0.25) (layer "F.Cu") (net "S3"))
 (arc (start 152.891988 131.513642) (mid 153.034439 131.169735) (end 153.378346 131.027284) (width 0.25) (layer "F.Cu") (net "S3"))
 (arc (start 146.407807 132.968362) (mid 146.750175 132.826549) (end 146.891988 132.484181) (width 0.25) (layer "F.Cu") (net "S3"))
 (arc (start 150.40563 132.972716) (mid 150.749537 132.830265) (end 150.891988 132.486358) (width 0.25) (layer "F.Cu") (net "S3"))
 (arc (start 152.40563 132.972716) (mid 152.749537 132.830265) (end 152.891988 132.486358) (width 0.25) (layer "F.Cu") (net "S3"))
 (arc (start 147.40563 131.027284) (mid 147.749537 131.169735) (end 147.891988 131.513642) (width 0.25) (layer "F.Cu") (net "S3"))
 (arc (start 149.40563 131.027284) (mid 149.749537 131.169735) (end 149.891988 131.513642) (width 0.25) (layer "F.Cu") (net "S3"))
 (arc (start 155.891988 131.515829) (mid 156.033798 131.85819) (end 156.376159 132) (width 0.25) (layer "F.Cu") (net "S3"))
 (arc (start 151.891988 132.486358) (mid 152.034439 132.830265) (end 152.378346 132.972716) (width 0.25) (layer "F.Cu") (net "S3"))
 (arc (start 146.891988 131.513642) (mid 147.034439 131.169735) (end 147.378346 131.027284) (width 0.25) (layer "F.Cu") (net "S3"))
 (arc (start 145.876169 132.484181) (mid 146.017982 132.826549) (end 146.36035 132.968362) (width 0.25) (layer "F.Cu") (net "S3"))
 (arc (start 150.891988 131.513642) (mid 151.034439 131.169735) (end 151.378346 131.027284) (width 0.25) (layer "F.Cu") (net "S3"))
 (arc (start 153.891988 132.486358) (mid 154.034439 132.830265) (end 154.378346 132.972716) (width 0.25) (layer "F.Cu") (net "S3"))
 (arc (start 154.891988 131.515829) (mid 155.033798 131.173468) (end 155.376159 131.031658) (width 0.25) (layer "F.Cu") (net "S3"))
 (arc (start 126.707107 135.707107) (mid 127.03153 135.92388) (end 127.414214 136) (width 0.25) (layer "F.Cu") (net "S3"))
 (arc (start 153.40563 131.027284) (mid 153.749537 131.169735) (end 153.891988 131.513642) (width 0.25) (layer "F.Cu") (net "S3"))
 (arc (start 123.585786 133) (mid 123.96847 133.07612) (end 124.292893 133.292893) (width 0.25) (layer "F.Cu") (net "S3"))
 (arc (start 148.891988 131.513642) (mid 149.034439 131.169735) (end 149.378346 131.027284) (width 0.25) (layer "F.Cu") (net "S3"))
 (arc (start 148.40563 132.972716) (mid 148.749537 132.830265) (end 148.891988 132.486358) (width 0.25) (layer "F.Cu") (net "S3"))
 (arc (start 151.40563 131.027284) (mid 151.749537 131.169735) (end 151.891988 131.513642) (width 0.25) (layer "F.Cu") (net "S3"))
 (arc (start 149.891988 132.486358) (mid 150.034439 132.830265) (end 150.378346 132.972716) (width 0.25) (layer "F.Cu") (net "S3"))
 (arc (start 145.391988 132) (mid 145.734356 132.141813) (end 145.876169 132.484181) (width 0.25) (layer "F.Cu") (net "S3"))
 (arc (start 147.891988 132.486358) (mid 148.034439 132.830265) (end 148.378346 132.972716) (width 0.25) (layer "F.Cu") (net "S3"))
 (arc (start 155.407817 131.031658) (mid 155.750178 131.173468) (end 155.891988 131.515829) (width 0.25) (layer "F.Cu") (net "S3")))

